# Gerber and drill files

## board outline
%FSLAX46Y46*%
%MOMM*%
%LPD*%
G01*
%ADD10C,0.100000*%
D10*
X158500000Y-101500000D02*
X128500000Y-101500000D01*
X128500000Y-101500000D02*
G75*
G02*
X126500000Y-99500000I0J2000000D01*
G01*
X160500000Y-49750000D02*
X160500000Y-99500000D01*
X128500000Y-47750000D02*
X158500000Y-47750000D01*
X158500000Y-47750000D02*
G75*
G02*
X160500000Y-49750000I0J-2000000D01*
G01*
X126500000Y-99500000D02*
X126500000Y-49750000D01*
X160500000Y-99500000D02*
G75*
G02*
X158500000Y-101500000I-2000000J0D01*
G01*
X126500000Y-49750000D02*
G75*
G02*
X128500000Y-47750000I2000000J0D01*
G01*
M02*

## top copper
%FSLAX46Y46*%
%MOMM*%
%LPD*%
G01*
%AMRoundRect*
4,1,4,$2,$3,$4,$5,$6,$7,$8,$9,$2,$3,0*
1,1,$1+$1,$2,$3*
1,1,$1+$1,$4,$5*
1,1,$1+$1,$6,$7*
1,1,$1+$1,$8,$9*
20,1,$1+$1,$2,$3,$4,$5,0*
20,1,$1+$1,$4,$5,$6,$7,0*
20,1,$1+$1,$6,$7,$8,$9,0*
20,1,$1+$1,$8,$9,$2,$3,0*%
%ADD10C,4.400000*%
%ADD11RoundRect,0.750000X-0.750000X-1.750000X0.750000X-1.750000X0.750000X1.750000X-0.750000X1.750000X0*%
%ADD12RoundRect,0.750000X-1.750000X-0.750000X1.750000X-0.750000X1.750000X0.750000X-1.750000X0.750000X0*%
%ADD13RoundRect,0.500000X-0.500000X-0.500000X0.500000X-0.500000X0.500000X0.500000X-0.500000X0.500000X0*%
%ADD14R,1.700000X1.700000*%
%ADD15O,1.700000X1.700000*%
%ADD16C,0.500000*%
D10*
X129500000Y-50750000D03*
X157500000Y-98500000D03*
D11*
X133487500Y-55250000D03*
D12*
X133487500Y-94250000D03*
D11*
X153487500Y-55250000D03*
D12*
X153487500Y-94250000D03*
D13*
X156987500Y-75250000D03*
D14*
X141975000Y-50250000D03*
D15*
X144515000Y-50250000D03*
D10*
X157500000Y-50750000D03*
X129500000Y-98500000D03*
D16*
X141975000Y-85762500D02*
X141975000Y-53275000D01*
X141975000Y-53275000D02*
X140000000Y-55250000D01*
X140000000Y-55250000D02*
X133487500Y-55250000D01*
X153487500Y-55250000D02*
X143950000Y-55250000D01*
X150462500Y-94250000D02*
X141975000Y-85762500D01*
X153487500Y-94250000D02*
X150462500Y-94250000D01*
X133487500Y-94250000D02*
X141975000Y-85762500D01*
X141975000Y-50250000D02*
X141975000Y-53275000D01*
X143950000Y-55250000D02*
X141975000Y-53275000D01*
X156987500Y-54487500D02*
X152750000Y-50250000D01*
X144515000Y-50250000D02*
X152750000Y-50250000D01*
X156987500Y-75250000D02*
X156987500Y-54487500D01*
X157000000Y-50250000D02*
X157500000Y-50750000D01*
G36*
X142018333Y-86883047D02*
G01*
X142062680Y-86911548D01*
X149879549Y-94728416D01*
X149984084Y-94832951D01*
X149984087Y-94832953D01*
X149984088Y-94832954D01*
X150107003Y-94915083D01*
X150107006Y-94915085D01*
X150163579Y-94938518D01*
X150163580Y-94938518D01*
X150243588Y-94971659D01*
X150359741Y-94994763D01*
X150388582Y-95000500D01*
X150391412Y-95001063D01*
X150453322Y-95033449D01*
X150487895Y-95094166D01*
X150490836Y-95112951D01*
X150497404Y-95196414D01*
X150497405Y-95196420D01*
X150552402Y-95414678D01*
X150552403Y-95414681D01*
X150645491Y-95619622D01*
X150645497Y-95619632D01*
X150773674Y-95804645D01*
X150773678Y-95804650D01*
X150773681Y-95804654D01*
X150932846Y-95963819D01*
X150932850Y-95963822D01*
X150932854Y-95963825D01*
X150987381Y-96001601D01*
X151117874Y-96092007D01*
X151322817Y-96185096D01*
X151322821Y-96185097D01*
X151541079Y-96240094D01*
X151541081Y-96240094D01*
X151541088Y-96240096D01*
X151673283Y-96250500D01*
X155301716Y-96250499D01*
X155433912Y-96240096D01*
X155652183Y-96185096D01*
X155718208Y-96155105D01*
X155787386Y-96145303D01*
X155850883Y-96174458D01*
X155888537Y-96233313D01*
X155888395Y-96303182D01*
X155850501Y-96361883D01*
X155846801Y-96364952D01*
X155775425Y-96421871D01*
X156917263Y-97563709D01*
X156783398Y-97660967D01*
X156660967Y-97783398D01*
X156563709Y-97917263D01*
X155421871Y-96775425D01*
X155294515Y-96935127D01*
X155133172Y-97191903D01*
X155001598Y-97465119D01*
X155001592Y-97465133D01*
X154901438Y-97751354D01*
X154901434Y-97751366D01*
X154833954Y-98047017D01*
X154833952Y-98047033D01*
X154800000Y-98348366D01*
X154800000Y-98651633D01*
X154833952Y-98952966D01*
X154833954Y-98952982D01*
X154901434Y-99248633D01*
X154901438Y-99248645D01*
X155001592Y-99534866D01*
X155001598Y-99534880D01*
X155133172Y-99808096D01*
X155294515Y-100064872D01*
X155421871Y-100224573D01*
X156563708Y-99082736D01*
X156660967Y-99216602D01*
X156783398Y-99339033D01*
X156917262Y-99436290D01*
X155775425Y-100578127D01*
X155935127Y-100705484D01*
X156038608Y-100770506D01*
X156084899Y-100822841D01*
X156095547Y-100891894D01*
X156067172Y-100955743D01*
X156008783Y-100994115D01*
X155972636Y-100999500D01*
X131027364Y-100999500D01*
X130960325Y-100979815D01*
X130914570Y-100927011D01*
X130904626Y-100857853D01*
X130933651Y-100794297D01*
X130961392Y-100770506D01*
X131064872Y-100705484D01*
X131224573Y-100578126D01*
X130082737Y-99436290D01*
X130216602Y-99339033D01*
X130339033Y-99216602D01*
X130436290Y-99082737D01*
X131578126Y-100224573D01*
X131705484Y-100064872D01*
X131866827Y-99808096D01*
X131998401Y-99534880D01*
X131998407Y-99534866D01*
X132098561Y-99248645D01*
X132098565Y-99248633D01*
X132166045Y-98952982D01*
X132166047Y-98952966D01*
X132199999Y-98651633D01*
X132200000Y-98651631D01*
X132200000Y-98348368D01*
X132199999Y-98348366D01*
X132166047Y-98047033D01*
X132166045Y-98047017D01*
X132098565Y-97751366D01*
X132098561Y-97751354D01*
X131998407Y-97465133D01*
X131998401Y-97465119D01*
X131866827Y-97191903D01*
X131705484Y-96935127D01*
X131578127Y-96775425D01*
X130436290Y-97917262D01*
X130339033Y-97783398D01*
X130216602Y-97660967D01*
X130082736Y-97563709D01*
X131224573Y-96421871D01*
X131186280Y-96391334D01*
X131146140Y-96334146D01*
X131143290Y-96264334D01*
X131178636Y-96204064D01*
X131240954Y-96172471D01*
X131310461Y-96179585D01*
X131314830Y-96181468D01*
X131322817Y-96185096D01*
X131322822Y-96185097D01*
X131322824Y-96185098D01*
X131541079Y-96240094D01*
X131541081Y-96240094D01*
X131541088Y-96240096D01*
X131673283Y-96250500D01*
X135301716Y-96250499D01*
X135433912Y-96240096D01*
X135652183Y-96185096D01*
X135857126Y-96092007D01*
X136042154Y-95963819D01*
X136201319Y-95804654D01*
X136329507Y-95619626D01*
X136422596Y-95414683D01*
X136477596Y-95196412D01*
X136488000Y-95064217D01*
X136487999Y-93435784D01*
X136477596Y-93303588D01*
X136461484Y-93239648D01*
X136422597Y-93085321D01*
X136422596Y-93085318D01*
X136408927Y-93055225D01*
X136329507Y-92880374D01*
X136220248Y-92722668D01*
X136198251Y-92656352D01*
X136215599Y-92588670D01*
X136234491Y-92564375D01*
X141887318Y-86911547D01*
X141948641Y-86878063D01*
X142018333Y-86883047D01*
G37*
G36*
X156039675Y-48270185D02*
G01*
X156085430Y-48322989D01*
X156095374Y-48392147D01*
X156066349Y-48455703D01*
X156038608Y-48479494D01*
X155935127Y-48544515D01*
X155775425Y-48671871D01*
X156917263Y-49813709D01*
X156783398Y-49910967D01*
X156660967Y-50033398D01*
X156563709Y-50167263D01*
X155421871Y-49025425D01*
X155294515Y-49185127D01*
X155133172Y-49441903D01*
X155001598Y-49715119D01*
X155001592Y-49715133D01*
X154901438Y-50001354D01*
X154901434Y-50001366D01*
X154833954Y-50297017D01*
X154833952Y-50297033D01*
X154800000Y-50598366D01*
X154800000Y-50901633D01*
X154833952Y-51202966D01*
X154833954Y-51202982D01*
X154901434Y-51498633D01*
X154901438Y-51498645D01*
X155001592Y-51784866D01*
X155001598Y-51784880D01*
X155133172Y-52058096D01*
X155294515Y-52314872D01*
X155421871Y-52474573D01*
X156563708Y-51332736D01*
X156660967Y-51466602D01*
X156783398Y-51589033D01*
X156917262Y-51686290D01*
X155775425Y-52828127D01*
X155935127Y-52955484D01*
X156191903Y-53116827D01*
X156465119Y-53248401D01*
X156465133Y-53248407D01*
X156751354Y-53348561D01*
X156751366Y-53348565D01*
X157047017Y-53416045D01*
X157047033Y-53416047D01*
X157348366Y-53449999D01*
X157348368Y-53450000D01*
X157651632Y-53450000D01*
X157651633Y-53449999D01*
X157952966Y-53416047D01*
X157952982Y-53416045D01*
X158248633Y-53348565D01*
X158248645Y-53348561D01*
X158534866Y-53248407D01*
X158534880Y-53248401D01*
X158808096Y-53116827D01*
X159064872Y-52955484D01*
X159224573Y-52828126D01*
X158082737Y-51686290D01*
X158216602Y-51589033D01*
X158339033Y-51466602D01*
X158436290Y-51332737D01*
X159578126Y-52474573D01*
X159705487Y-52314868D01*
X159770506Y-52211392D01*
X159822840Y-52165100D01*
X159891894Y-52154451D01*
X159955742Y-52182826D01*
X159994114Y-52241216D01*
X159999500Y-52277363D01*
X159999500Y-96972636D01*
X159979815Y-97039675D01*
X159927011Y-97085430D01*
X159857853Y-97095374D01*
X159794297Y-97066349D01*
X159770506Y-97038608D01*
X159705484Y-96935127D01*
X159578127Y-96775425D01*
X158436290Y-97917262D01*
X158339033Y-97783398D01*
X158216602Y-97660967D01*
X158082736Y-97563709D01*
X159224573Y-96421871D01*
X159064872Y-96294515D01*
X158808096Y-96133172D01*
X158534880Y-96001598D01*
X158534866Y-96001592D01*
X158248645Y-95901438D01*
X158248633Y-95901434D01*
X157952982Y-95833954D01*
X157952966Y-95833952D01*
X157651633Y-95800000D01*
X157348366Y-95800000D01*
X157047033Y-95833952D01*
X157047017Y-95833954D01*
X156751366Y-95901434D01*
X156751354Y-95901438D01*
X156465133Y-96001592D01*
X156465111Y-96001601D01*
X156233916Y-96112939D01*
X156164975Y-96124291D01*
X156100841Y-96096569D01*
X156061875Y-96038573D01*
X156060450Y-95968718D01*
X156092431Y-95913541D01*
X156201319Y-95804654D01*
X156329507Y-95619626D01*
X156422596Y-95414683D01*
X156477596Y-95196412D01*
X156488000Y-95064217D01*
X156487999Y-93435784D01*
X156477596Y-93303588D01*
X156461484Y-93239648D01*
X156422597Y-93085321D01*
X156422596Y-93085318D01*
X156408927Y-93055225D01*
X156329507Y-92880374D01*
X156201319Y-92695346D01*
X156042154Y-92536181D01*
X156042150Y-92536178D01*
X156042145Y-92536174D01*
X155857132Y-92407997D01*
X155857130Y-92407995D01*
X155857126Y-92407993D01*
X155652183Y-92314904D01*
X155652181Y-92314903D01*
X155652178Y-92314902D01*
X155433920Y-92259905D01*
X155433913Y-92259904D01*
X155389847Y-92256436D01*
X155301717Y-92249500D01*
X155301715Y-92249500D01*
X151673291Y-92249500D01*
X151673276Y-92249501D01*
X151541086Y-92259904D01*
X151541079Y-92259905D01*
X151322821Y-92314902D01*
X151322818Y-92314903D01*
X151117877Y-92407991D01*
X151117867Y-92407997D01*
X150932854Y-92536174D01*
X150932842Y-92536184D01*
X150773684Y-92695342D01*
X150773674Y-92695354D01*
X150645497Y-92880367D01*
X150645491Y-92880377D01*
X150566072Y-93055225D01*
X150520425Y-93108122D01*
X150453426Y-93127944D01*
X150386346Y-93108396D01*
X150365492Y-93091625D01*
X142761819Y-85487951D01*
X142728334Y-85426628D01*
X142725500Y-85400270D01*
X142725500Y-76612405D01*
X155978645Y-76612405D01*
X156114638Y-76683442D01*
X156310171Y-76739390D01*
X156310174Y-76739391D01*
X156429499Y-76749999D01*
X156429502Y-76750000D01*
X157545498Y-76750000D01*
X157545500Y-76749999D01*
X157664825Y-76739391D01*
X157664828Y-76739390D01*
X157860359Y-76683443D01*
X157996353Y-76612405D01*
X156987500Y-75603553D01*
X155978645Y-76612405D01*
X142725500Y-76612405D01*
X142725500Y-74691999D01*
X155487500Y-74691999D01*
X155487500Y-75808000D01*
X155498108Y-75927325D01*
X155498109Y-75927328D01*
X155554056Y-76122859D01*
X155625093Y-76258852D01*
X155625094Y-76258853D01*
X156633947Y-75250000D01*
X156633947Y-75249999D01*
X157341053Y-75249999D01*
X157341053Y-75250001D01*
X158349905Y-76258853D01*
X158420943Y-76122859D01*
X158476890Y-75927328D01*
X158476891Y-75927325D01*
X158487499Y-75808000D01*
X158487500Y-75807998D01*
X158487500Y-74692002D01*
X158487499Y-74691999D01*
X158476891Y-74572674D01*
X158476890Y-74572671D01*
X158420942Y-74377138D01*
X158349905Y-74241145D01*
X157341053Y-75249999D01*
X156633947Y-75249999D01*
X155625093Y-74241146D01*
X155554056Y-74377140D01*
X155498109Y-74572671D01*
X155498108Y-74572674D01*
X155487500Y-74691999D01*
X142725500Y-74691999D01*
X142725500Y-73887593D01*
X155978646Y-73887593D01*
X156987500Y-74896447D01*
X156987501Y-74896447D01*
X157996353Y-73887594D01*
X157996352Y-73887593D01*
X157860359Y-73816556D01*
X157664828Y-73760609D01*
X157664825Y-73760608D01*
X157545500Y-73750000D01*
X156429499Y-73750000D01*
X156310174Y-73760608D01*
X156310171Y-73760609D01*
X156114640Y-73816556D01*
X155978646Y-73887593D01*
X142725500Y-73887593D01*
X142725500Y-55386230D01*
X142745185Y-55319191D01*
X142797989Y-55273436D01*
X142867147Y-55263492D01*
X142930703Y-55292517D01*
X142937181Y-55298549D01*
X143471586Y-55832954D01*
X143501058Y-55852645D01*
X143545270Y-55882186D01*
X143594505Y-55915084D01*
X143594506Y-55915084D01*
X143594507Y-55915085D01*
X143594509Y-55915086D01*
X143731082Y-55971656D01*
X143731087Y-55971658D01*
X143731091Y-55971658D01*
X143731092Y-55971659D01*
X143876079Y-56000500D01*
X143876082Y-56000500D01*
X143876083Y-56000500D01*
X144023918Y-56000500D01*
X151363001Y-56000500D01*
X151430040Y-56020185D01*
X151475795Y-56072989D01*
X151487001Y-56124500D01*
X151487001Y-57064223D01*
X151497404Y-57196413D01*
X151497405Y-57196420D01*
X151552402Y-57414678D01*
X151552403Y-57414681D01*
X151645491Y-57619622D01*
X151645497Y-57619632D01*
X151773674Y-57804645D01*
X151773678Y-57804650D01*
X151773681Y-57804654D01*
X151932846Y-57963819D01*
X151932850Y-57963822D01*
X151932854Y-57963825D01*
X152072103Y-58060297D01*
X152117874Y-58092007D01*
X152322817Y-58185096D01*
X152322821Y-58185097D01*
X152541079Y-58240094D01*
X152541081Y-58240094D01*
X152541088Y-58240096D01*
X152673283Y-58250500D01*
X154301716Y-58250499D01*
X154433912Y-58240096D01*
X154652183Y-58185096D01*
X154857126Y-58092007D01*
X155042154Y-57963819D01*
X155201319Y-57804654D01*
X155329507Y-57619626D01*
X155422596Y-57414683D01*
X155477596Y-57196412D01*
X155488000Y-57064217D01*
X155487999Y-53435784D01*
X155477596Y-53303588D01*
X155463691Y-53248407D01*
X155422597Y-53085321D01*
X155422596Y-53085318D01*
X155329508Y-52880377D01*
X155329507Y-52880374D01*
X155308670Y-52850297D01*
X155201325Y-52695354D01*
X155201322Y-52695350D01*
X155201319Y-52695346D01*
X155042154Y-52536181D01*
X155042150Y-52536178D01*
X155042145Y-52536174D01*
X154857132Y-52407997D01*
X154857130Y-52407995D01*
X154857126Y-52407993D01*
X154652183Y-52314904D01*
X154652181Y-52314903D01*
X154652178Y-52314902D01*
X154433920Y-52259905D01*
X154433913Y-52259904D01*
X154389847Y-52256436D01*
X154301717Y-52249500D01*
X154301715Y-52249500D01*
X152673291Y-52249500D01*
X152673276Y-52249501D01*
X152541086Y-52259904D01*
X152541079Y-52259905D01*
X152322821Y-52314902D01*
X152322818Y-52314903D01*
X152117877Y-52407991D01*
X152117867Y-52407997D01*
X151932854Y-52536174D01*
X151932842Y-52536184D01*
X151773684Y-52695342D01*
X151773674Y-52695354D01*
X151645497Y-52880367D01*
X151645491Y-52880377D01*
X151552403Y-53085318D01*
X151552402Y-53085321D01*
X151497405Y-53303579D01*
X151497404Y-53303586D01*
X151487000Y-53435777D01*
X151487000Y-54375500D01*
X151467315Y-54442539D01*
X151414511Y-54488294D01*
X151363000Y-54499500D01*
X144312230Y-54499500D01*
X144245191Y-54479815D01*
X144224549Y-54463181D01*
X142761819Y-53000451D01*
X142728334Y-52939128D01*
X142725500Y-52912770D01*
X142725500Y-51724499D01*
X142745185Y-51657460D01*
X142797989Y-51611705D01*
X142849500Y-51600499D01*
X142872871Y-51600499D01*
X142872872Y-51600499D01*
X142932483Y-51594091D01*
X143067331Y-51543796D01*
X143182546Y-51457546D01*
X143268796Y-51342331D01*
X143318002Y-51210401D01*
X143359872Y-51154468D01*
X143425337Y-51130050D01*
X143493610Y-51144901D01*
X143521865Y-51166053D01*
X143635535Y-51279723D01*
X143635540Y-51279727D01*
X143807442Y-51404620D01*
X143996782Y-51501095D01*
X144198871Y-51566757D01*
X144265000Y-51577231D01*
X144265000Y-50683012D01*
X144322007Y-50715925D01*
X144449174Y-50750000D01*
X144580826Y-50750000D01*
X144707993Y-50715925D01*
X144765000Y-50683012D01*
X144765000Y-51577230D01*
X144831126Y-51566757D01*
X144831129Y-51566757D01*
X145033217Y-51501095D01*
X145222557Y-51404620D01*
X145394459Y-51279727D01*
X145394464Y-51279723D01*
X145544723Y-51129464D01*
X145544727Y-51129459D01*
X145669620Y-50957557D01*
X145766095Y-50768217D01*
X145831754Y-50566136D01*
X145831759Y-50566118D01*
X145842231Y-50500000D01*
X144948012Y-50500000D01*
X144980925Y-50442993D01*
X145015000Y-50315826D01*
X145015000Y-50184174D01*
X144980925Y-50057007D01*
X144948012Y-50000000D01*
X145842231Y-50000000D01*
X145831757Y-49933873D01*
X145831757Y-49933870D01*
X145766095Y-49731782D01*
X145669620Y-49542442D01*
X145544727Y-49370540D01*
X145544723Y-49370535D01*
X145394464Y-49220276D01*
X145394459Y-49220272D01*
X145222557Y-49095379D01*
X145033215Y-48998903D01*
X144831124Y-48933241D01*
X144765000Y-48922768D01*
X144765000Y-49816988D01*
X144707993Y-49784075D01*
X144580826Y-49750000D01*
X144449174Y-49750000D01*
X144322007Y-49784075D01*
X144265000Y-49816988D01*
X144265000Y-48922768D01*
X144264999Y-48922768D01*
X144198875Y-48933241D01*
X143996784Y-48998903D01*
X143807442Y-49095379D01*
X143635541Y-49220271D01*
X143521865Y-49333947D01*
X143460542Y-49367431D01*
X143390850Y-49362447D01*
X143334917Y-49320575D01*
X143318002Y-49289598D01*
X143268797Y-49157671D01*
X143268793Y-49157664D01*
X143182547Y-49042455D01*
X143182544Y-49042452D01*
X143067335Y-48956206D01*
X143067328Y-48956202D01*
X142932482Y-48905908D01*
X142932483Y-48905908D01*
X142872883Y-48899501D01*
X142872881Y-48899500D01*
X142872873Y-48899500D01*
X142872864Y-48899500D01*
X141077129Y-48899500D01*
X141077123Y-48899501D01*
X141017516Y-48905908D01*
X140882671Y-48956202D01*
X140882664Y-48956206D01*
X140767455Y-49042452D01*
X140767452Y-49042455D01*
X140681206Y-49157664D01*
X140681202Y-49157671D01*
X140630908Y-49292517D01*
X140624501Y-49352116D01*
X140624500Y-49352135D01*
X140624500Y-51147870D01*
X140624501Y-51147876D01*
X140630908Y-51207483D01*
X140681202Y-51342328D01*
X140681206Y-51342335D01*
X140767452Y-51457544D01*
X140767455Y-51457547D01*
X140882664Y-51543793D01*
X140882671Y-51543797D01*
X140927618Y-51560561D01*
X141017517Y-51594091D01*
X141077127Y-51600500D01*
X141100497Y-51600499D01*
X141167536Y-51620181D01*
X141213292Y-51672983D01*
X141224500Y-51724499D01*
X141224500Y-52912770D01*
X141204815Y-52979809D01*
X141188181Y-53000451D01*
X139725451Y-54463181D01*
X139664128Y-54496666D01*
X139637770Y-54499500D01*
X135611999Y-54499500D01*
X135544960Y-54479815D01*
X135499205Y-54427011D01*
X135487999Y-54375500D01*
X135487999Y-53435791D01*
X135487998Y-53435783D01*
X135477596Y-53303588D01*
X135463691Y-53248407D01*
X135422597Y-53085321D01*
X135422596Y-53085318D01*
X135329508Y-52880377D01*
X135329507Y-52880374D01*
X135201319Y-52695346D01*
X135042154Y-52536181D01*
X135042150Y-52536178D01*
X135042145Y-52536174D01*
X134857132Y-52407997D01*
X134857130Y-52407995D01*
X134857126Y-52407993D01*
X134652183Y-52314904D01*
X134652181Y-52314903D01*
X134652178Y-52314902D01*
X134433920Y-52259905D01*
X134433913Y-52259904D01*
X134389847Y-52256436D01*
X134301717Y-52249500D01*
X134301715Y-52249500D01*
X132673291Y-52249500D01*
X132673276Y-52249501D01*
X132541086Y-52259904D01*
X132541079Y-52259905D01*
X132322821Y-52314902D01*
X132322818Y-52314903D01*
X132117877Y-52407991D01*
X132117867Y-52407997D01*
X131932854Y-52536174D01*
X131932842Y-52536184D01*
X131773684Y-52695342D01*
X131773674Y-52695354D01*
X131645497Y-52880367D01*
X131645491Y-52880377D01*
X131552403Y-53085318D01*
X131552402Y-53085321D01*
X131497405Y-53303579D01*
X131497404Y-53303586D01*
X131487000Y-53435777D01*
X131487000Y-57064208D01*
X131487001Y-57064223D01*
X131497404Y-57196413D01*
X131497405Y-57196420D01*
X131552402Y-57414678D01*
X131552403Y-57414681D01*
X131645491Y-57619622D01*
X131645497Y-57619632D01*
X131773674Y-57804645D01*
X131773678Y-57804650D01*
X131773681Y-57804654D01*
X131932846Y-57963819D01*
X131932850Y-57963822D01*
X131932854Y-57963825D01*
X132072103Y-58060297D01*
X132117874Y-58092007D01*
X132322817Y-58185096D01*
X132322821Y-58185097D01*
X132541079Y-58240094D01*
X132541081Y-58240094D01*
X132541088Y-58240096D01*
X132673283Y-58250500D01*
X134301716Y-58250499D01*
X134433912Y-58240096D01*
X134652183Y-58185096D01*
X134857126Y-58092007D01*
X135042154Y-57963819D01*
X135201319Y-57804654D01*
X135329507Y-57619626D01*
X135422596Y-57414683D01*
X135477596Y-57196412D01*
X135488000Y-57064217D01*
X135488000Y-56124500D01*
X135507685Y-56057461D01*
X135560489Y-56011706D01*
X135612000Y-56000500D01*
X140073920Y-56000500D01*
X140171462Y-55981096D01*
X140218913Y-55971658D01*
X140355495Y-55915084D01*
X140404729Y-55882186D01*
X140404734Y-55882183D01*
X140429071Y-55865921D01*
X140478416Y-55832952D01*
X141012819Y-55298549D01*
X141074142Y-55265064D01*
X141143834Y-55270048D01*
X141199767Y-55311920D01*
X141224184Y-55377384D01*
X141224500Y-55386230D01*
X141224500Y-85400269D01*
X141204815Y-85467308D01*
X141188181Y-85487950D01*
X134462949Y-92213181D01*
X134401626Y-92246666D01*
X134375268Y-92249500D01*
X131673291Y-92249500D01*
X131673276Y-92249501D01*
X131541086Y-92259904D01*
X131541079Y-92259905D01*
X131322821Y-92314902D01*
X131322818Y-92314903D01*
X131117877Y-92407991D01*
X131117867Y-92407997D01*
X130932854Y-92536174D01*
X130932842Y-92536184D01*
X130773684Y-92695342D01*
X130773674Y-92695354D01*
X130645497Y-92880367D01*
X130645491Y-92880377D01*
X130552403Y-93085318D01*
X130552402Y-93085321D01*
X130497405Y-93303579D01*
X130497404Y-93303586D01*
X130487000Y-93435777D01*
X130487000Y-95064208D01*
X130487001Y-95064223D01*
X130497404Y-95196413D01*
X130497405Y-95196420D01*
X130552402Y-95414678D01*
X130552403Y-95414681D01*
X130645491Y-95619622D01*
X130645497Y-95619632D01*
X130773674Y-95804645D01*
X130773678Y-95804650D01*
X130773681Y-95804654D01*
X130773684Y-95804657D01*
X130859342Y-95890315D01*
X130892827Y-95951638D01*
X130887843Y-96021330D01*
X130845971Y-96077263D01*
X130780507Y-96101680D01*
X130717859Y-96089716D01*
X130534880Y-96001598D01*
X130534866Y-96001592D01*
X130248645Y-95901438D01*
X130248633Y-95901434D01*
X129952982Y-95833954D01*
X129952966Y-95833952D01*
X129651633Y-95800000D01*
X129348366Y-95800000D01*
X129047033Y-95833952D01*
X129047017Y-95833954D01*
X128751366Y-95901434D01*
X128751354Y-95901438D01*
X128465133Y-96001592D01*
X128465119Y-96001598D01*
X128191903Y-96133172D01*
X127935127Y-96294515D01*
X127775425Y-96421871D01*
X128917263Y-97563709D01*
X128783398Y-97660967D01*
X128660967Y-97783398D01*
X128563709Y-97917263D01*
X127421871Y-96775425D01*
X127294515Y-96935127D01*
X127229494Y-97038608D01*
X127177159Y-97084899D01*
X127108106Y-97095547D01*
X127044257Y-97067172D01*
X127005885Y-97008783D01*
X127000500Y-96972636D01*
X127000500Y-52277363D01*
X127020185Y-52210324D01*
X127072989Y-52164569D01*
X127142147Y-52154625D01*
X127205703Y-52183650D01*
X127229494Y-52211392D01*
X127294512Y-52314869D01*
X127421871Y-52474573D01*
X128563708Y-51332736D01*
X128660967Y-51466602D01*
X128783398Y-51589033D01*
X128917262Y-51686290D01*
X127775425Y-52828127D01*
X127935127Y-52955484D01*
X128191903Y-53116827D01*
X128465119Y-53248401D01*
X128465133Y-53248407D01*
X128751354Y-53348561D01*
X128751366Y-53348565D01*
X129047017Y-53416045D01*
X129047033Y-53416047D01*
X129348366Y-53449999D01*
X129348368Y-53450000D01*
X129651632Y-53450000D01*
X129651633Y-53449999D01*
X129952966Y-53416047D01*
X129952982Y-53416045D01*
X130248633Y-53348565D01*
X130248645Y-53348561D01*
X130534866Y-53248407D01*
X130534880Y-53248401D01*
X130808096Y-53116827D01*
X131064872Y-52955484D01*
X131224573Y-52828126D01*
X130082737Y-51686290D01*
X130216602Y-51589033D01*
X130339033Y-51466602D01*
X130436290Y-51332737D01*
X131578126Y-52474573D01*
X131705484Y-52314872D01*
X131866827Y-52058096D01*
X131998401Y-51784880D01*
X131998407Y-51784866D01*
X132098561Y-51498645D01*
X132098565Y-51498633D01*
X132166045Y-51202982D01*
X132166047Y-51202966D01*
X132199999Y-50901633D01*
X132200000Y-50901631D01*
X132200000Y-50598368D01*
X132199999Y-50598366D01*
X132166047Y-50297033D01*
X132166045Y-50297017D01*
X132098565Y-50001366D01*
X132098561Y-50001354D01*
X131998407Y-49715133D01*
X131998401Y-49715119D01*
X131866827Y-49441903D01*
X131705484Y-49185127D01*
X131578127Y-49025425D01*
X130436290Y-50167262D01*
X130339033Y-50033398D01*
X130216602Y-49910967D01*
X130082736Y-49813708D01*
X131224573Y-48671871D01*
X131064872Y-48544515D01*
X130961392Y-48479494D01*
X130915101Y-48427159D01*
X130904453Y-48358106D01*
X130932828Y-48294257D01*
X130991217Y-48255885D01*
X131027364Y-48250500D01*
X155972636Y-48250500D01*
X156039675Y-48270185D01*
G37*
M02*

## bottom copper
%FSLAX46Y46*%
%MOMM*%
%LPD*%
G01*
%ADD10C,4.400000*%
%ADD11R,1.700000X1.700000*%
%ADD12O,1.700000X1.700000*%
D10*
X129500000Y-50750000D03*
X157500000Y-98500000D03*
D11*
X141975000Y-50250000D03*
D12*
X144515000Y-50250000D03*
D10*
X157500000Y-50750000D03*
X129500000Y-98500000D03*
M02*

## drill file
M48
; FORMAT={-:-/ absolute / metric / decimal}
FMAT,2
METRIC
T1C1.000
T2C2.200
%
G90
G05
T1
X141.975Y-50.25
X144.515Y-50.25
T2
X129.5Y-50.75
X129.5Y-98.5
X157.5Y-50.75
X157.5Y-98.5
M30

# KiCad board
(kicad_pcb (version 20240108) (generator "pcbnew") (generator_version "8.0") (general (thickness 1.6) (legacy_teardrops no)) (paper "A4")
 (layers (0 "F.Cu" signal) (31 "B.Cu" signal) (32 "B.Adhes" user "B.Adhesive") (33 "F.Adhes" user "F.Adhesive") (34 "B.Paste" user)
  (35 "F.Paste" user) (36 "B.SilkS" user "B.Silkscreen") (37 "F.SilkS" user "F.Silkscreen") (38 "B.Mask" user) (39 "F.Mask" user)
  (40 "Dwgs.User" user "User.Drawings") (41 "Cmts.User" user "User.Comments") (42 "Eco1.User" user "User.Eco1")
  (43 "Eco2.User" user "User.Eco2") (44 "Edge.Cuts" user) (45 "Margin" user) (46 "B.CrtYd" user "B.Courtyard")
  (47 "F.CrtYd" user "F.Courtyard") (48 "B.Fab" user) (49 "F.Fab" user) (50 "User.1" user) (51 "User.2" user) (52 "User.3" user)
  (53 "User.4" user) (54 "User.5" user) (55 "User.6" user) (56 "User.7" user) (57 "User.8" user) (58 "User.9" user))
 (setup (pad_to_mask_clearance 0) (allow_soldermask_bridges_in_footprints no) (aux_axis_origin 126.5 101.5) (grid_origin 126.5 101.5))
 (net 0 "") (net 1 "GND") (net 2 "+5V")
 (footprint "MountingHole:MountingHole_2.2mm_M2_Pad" (layer "F.Cu") (at 129.5 50.75)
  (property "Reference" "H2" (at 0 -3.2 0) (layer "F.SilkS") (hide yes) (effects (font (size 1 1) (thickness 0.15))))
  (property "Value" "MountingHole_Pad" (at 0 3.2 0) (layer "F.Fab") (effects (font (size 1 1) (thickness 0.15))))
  (pad "1" thru_hole circle (at 0 0) (size 4.4 4.4) (drill 2.2) (layers "*.Cu" "*.Mask") (remove_unused_layers no) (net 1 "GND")))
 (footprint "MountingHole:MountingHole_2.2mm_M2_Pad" (layer "F.Cu") (at 157.5 98.5)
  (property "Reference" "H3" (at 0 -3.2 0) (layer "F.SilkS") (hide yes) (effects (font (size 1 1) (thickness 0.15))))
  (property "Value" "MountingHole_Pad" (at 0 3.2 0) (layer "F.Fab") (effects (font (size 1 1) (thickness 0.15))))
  (pad "1" thru_hole circle (at 0 0) (size 4.4 4.4) (drill 2.2) (layers "*.Cu" "*.Mask") (remove_unused_layers no) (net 1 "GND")))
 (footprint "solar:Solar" (layer "F.Cu") (at 133.9875 95.25)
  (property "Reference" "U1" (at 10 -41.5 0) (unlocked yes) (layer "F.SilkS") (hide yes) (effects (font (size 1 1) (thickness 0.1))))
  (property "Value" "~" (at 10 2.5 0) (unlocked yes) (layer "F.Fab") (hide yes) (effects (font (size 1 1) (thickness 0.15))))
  (pad "1" smd roundrect (at -0.5 -40) (size 3 5) (layers "F.Cu" "F.Paste" "F.Mask") (roundrect_rratio 0.25) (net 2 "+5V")
   (thermal_bridge_angle 45))
  (pad "1" smd roundrect (at -0.5 -1) (size 5 3) (layers "F.Cu" "F.Paste" "F.Mask") (roundrect_rratio 0.25) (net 2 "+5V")
   (thermal_bridge_angle 45))
  (pad "1" smd roundrect (at 19.5 -40) (size 3 5) (layers "F.Cu" "F.Paste" "F.Mask") (roundrect_rratio 0.25) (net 2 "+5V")
   (thermal_bridge_angle 45))
  (pad "1" smd roundrect (at 19.5 -1) (size 5 3) (layers "F.Cu" "F.Paste" "F.Mask") (roundrect_rratio 0.25) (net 2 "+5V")
   (thermal_bridge_angle 45))
  (pad "2" smd roundrect (at 23 -20) (size 2 2) (layers "F.Cu" "F.Paste" "F.Mask") (roundrect_rratio 0.25) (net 1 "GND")
   (thermal_bridge_angle 45)))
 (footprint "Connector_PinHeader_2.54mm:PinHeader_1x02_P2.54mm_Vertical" (layer "F.Cu") (at 141.975 50.25 90)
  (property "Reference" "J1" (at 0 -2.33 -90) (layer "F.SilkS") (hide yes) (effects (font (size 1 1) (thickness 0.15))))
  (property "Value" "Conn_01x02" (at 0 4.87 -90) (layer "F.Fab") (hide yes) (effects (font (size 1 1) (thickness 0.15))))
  (pad "1" thru_hole rect (at 0 0 90) (size 1.7 1.7) (drill 1) (layers "*.Cu" "*.Mask") (remove_unused_layers no) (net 2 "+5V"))
  (pad "2" thru_hole oval (at 0 2.54 90) (size 1.7 1.7) (drill 1) (layers "*.Cu" "*.Mask") (remove_unused_layers no) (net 1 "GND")))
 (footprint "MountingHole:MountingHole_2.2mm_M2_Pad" (layer "F.Cu") (at 157.5 50.75)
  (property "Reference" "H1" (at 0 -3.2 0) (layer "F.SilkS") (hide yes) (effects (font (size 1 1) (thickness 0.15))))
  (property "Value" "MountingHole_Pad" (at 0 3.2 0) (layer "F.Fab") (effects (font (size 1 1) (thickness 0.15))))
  (pad "1" thru_hole circle (at 0 0) (size 4.4 4.4) (drill 2.2) (layers "*.Cu" "*.Mask") (remove_unused_layers no) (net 1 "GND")))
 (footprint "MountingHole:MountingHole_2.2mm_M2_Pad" (layer "F.Cu") (at 129.5 98.5)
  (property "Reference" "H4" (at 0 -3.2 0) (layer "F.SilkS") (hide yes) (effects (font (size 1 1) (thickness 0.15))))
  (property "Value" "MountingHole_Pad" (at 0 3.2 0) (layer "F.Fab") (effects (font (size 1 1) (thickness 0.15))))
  (pad "1" thru_hole circle (at 0 0) (size 4.4 4.4) (drill 2.2) (layers "*.Cu" "*.Mask") (remove_unused_layers no) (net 1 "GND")))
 (gr_line (start 158.5 101.5) (end 128.5 101.5) (stroke (width 0.1) (type default)) (layer "Edge.Cuts"))
 (gr_arc (start 128.5 101.5) (mid 127.085786 100.914214) (end 126.5 99.5) (stroke (width 0.1) (type default)) (layer "Edge.Cuts"))
 (gr_line (start 160.5 49.75) (end 160.5 99.5) (stroke (width 0.1) (type default)) (layer "Edge.Cuts"))
 (gr_line (start 128.5 47.75) (end 158.5 47.75) (stroke (width 0.1) (type default)) (layer "Edge.Cuts"))
 (gr_arc (start 158.5 47.75) (mid 159.914214 48.335786) (end 160.5 49.75) (stroke (width 0.1) (type default)) (layer "Edge.Cuts"))
 (gr_line (start 126.5 99.5) (end 126.5 49.75) (stroke (width 0.1) (type default)) (layer "Edge.Cuts"))
 (gr_arc (start 160.5 99.5) (mid 159.914214 100.914214) (end 158.5 101.5) (stroke (width 0.1) (type default)) (layer "Edge.Cuts"))
 (gr_arc (start 126.5 49.75) (mid 127.085786 48.335786) (end 128.5 47.75) (stroke (width 0.1) (type default)) (layer "Edge.Cuts"))
 (segment (start 141.975 85.7625) (end 141.975 53.275) (width 0.5) (layer "F.Cu") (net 2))
 (segment (start 141.975 53.275) (end 140 55.25) (width 0.5) (layer "F.Cu") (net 2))
 (segment (start 140 55.25) (end 133.4875 55.25) (width 0.5) (layer "F.Cu") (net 2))
 (segment (start 153.4875 55.25) (end 143.95 55.25) (width 0.5) (layer "F.Cu") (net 2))
 (segment (start 150.4625 94.25) (end 141.975 85.7625) (width 0.5) (layer "F.Cu") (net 2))
 (segment (start 153.4875 94.25) (end 150.4625 94.25) (width 0.5) (layer "F.Cu") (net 2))
 (segment (start 133.4875 94.25) (end 141.975 85.7625) (width 0.5) (layer "F.Cu") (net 2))
 (segment (start 141.975 50.25) (end 141.975 53.275) (width 0.5) (layer "F.Cu") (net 2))
 (segment (start 143.95 55.25) (end 141.975 53.275) (width 0.5) (layer "F.Cu") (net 2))
 (segment (start 156.9875 54.4875) (end 152.75 50.25) (width 0.5) (layer "F.Cu") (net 1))
 (segment (start 144.515 50.25) (end 152.75 50.25) (width 0.5) (layer "F.Cu") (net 1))
 (segment (start 156.9875 75.25) (end 156.9875 54.4875) (width 0.5) (layer "F.Cu") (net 1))
 (segment (start 157 50.25) (end 157.5 50.75) (width 0.5) (layer "F.Cu") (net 1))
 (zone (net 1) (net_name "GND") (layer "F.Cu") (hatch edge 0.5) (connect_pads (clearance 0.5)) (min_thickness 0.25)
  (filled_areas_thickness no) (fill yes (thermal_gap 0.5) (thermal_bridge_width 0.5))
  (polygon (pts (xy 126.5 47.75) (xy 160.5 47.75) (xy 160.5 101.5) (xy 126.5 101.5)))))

